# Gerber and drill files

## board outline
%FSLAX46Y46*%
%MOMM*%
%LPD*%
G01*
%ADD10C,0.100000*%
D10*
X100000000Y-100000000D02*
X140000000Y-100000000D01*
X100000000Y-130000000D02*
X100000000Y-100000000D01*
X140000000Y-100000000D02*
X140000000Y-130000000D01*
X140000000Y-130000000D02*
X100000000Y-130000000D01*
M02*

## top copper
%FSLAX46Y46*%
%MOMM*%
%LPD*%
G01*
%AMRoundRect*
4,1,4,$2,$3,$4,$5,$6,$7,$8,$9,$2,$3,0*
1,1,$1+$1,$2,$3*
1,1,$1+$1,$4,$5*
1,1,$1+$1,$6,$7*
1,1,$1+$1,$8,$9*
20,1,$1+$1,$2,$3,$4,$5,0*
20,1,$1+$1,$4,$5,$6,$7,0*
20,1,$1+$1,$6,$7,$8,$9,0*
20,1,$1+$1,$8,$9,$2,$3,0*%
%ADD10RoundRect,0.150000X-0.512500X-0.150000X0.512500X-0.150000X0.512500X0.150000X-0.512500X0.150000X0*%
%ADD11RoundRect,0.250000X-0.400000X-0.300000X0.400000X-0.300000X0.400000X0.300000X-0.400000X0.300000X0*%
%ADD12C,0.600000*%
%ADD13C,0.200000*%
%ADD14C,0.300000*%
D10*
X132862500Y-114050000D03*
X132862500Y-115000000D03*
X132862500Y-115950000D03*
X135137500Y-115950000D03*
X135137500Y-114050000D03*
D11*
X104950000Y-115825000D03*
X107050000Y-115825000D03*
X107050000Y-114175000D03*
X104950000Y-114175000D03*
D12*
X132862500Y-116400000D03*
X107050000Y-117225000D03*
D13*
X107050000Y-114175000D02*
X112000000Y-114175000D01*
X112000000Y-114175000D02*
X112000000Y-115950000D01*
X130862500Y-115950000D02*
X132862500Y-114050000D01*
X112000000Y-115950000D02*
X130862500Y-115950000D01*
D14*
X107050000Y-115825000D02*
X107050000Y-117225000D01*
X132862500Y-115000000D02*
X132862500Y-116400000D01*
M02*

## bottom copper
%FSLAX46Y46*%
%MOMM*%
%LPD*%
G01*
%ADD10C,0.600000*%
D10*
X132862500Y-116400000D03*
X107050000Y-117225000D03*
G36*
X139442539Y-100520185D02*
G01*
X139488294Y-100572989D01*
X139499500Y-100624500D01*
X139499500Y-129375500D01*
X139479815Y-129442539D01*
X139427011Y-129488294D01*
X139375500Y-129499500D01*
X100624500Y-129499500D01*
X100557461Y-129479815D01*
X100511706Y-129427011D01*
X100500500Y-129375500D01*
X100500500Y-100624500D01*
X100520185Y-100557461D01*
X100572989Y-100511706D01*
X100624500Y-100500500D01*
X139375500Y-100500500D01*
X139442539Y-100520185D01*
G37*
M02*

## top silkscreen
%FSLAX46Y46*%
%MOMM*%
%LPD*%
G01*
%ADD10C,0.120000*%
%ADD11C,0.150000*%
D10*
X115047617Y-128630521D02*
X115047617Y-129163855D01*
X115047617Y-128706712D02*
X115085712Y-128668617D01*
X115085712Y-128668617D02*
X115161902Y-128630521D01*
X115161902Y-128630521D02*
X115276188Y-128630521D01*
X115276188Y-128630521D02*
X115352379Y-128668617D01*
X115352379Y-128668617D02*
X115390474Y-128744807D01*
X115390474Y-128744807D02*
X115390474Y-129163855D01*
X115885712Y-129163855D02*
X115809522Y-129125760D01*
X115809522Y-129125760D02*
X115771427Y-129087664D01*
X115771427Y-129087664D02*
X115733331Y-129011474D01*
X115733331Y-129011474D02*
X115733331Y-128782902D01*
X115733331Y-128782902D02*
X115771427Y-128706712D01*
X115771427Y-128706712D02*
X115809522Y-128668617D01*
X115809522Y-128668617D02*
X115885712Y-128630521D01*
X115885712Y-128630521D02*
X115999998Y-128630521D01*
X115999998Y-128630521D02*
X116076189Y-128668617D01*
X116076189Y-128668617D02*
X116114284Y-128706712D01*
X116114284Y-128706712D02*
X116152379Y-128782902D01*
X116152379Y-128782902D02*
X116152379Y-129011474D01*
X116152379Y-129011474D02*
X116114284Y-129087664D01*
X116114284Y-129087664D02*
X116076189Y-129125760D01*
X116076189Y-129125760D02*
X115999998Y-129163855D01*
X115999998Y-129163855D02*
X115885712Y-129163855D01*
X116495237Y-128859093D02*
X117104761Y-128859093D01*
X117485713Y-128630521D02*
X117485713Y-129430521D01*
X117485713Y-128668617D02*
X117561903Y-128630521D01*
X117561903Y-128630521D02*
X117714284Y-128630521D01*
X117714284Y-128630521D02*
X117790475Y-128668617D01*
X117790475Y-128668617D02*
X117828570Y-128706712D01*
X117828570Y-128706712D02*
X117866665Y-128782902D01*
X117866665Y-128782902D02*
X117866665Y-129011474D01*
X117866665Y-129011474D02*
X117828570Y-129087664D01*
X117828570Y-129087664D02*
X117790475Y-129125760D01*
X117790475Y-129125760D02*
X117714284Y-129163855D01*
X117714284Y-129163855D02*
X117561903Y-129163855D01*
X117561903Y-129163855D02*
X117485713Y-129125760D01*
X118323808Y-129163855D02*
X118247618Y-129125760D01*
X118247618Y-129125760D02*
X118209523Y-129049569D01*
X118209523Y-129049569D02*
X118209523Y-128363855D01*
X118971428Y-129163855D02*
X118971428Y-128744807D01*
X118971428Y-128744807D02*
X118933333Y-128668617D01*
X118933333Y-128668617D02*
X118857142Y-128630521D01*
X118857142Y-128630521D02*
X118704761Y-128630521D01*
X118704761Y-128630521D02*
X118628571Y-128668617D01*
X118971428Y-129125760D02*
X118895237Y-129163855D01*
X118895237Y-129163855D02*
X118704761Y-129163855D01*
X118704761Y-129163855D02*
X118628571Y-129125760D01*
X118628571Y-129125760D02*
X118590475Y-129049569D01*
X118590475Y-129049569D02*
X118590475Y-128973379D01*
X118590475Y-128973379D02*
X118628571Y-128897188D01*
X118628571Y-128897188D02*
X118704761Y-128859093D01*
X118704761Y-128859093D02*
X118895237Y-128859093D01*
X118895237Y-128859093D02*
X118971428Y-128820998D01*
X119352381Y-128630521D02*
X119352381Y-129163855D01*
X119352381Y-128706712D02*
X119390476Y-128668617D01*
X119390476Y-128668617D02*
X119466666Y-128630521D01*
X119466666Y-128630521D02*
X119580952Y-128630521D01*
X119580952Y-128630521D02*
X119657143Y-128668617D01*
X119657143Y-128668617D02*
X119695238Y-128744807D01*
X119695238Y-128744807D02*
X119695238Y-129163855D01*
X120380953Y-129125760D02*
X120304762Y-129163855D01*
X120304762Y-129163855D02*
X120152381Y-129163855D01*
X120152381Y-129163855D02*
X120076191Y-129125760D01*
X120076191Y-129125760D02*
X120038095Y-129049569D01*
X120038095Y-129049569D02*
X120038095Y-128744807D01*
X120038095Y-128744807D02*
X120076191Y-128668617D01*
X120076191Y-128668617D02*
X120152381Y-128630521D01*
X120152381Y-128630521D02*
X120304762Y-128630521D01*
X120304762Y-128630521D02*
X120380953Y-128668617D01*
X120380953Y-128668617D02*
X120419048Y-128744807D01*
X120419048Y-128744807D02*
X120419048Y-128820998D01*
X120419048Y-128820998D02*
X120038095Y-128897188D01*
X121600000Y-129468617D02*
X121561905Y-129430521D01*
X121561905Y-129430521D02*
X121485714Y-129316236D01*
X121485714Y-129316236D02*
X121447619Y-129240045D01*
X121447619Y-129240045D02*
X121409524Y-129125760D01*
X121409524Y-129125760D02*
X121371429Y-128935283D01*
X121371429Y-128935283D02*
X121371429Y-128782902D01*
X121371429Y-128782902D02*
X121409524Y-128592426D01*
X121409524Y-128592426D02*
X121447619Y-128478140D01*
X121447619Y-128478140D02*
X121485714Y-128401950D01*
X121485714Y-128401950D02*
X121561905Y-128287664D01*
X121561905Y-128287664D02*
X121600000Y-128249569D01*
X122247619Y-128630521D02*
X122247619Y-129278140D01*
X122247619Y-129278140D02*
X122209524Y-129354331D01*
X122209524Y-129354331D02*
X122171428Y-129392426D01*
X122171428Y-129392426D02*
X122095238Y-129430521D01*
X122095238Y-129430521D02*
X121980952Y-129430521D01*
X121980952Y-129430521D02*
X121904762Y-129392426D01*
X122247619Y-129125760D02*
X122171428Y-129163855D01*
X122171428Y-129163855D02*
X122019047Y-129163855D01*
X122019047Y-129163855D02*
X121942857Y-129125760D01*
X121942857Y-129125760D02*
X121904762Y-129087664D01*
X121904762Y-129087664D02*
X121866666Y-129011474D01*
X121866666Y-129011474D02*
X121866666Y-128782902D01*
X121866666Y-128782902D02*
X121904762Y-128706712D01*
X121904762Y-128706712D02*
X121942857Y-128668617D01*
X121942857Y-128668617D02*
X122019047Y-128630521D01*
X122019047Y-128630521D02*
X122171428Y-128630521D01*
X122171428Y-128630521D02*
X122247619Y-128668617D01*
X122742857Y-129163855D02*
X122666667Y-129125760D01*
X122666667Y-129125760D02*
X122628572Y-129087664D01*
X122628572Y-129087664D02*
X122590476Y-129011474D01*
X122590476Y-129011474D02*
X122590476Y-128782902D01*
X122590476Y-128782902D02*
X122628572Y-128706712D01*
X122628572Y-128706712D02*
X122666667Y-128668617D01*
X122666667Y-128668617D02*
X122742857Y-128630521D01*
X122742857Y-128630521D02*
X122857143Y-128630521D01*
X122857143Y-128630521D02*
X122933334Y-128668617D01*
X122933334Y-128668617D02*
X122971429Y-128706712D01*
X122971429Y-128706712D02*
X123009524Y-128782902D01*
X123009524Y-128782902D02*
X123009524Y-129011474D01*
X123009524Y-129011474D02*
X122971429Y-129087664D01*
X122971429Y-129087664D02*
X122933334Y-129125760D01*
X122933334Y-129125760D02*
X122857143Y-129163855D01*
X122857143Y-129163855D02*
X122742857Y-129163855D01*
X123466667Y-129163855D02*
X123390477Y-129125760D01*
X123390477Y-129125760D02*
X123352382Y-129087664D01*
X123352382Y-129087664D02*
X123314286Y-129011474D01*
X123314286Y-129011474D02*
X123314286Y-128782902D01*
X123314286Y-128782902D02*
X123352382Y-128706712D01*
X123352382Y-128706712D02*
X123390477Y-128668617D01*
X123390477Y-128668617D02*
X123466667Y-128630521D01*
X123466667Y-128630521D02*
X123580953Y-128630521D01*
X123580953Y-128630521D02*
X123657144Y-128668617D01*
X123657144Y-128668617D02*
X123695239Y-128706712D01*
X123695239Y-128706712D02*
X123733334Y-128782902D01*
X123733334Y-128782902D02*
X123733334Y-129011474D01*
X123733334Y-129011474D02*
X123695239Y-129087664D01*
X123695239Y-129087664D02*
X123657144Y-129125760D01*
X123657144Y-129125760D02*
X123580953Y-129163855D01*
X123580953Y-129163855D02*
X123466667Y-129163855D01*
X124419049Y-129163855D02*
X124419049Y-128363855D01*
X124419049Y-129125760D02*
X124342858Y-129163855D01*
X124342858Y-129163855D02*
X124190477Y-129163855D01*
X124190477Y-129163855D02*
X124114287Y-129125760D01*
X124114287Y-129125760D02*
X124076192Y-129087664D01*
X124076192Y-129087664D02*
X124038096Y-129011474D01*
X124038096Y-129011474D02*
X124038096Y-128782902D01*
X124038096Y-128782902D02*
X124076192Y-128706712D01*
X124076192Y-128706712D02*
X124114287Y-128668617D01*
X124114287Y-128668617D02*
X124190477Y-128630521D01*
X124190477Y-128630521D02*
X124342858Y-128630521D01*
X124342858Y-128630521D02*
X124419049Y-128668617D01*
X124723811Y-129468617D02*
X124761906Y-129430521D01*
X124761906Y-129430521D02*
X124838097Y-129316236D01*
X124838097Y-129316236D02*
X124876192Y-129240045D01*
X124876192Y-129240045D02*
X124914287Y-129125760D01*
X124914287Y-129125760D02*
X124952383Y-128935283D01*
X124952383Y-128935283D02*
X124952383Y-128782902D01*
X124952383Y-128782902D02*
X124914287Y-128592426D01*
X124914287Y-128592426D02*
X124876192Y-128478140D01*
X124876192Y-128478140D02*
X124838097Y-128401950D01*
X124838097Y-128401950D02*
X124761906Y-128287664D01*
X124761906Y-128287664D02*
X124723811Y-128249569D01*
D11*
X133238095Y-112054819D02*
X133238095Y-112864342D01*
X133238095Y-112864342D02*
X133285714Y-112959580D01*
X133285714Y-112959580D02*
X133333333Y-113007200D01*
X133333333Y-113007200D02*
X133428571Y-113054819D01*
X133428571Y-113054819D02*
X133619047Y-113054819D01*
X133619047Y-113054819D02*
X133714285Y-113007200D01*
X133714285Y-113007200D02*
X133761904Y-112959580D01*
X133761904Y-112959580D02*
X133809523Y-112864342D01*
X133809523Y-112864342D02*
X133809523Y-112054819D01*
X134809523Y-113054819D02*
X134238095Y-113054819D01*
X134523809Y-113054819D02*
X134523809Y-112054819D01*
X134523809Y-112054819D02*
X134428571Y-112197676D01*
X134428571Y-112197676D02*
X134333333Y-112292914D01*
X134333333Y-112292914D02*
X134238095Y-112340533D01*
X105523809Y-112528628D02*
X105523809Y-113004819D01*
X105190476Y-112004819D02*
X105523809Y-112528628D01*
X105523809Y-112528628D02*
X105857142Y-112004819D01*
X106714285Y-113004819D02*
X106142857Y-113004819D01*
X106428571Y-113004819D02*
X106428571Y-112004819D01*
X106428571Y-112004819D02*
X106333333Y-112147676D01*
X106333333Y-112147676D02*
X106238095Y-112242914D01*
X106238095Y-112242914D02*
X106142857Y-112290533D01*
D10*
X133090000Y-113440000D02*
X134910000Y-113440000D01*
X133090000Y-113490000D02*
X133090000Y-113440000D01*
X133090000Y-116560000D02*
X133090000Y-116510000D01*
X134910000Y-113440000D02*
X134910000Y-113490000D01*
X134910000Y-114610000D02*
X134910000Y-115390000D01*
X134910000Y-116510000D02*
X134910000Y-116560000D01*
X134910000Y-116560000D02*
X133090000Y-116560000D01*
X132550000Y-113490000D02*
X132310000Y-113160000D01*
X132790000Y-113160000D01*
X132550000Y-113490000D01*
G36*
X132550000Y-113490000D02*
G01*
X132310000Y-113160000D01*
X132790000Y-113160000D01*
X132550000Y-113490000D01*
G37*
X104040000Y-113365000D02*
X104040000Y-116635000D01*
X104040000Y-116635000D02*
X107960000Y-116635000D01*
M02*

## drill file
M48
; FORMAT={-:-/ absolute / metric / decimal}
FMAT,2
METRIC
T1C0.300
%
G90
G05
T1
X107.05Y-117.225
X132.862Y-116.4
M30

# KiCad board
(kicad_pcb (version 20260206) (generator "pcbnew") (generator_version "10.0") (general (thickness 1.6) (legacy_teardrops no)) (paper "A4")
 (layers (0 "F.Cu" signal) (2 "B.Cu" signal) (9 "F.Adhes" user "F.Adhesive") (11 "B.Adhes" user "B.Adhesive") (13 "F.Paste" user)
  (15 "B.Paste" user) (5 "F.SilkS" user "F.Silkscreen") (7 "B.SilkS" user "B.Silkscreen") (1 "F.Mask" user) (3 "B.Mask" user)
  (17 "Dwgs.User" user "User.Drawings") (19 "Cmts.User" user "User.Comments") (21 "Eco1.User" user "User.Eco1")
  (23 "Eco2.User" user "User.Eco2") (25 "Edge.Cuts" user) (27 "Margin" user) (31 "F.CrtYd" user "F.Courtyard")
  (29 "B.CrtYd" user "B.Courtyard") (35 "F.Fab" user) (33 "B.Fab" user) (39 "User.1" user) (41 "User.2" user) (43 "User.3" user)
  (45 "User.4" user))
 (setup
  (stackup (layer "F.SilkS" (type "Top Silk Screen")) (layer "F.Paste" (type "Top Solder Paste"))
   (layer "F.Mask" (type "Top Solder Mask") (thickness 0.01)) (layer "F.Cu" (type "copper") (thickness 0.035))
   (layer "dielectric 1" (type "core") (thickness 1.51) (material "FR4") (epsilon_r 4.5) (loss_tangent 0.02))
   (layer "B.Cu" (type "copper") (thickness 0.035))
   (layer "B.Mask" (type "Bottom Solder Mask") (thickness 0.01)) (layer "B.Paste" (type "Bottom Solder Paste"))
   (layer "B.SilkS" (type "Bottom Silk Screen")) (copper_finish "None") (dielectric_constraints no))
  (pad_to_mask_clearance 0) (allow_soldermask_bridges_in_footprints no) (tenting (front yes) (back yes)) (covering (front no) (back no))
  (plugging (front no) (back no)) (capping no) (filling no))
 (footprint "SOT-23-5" (layer "F.Cu") (at 134 115)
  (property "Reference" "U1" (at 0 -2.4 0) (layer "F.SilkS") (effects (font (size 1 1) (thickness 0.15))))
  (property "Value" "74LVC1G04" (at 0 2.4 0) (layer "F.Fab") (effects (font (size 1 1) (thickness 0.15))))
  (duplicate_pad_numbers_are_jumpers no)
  (fp_line (start -0.91 -1.56) (end 0.91 -1.56) (stroke (width 0.12) (type solid)) (layer "F.SilkS"))
  (fp_line (start -0.91 -1.51) (end -0.91 -1.56) (stroke (width 0.12) (type solid)) (layer "F.SilkS"))
  (fp_line (start -0.91 1.56) (end -0.91 1.51) (stroke (width 0.12) (type solid)) (layer "F.SilkS"))
  (fp_line (start 0.91 -1.56) (end 0.91 -1.51) (stroke (width 0.12) (type solid)) (layer "F.SilkS"))
  (fp_line (start 0.91 -0.39) (end 0.91 0.39) (stroke (width 0.12) (type solid)) (layer "F.SilkS"))
  (fp_line (start 0.91 1.51) (end 0.91 1.56) (stroke (width 0.12) (type solid)) (layer "F.SilkS"))
  (fp_line (start 0.91 1.56) (end -0.91 1.56) (stroke (width 0.12) (type solid)) (layer "F.SilkS"))
  (fp_poly (pts (xy -1.45 -1.51) (xy -1.69 -1.84) (xy -1.21 -1.84)) (stroke (width 0.12) (type solid)) (fill yes) (layer "F.SilkS"))
  (pad "1" smd roundrect (at -1.1375 -0.95) (size 1.325 0.6) (layers "F.Cu" "F.Mask" "F.Paste") (roundrect_rratio 0.25) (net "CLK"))
  (pad "2" smd roundrect (at -1.1375 0) (size 1.325 0.6) (layers "F.Cu" "F.Mask" "F.Paste") (roundrect_rratio 0.25) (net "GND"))
  (pad "3" smd roundrect (at -1.1375 0.95) (size 1.325 0.6) (layers "F.Cu" "F.Mask" "F.Paste") (roundrect_rratio 0.25))
  (pad "4" smd roundrect (at 1.1375 0.95) (size 1.325 0.6) (layers "F.Cu" "F.Mask" "F.Paste") (roundrect_rratio 0.25))
  (pad "5" smd roundrect (at 1.1375 -0.95) (size 1.325 0.6) (layers "F.Cu" "F.Mask" "F.Paste") (roundrect_rratio 0.25) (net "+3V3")))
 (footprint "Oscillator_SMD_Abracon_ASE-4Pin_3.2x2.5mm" (layer "F.Cu") (at 106 115)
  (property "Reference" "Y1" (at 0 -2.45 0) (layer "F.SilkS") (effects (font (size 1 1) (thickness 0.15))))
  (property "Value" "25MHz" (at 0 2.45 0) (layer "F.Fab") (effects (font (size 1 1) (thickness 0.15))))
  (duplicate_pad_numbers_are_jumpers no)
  (fp_line (start -1.96 -1.635) (end -1.96 1.635) (stroke (width 0.12) (type solid)) (layer "F.SilkS"))
  (fp_line (start -1.96 1.635) (end 1.96 1.635) (stroke (width 0.12) (type solid)) (layer "F.SilkS"))
  (pad "1" smd roundrect (at -1.05 0.825) (size 1.3 1.1) (layers "F.Cu" "F.Mask" "F.Paste") (roundrect_rratio 0.227273) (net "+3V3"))
  (pad "2" smd roundrect (at 1.05 0.825) (size 1.3 1.1) (layers "F.Cu" "F.Mask" "F.Paste") (roundrect_rratio 0.227273) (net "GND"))
  (pad "3" smd roundrect (at 1.05 -0.825) (size 1.3 1.1) (layers "F.Cu" "F.Mask" "F.Paste") (roundrect_rratio 0.227273) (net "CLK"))
  (pad "4" smd roundrect (at -1.05 -0.825) (size 1.3 1.1) (layers "F.Cu" "F.Mask" "F.Paste") (roundrect_rratio 0.227273) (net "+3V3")))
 (gr_line (start 100 100) (end 140 100) (stroke (width 0.1) (type default)) (layer "Edge.Cuts"))
 (gr_line (start 100 130) (end 100 100) (stroke (width 0.1) (type default)) (layer "Edge.Cuts"))
 (gr_line (start 140 100) (end 140 130) (stroke (width 0.1) (type default)) (layer "Edge.Cuts"))
 (gr_line (start 140 130) (end 100 130) (stroke (width 0.1) (type default)) (layer "Edge.Cuts"))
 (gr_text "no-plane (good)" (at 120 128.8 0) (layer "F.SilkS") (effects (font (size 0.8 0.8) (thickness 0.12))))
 (segment (start 107.05 114.175) (end 112 114.175) (width 0.2) (layer "F.Cu") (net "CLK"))
 (segment (start 112 114.175) (end 112 115.95) (width 0.2) (layer "F.Cu") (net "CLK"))
 (segment (start 130.8625 115.95) (end 132.8625 114.05) (width 0.2) (layer "F.Cu") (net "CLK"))
 (segment (start 112 115.95) (end 130.8625 115.95) (width 0.2) (layer "F.Cu") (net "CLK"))
 (segment (start 107.05 115.825) (end 107.05 117.225) (width 0.3) (layer "F.Cu") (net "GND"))
 (segment (start 132.8625 115) (end 132.8625 116.4) (width 0.3) (layer "F.Cu") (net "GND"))
 (via (at 132.8625 116.4) (size 0.6) (drill 0.3) (layers "F.Cu" "B.Cu") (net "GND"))
 (via (at 107.05 117.225) (size 0.6) (drill 0.3) (layers "F.Cu" "B.Cu") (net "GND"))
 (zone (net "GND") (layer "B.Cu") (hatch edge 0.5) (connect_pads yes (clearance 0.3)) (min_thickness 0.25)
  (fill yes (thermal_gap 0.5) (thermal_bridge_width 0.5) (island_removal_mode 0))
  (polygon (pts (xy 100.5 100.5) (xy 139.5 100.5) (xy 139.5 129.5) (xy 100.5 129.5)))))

